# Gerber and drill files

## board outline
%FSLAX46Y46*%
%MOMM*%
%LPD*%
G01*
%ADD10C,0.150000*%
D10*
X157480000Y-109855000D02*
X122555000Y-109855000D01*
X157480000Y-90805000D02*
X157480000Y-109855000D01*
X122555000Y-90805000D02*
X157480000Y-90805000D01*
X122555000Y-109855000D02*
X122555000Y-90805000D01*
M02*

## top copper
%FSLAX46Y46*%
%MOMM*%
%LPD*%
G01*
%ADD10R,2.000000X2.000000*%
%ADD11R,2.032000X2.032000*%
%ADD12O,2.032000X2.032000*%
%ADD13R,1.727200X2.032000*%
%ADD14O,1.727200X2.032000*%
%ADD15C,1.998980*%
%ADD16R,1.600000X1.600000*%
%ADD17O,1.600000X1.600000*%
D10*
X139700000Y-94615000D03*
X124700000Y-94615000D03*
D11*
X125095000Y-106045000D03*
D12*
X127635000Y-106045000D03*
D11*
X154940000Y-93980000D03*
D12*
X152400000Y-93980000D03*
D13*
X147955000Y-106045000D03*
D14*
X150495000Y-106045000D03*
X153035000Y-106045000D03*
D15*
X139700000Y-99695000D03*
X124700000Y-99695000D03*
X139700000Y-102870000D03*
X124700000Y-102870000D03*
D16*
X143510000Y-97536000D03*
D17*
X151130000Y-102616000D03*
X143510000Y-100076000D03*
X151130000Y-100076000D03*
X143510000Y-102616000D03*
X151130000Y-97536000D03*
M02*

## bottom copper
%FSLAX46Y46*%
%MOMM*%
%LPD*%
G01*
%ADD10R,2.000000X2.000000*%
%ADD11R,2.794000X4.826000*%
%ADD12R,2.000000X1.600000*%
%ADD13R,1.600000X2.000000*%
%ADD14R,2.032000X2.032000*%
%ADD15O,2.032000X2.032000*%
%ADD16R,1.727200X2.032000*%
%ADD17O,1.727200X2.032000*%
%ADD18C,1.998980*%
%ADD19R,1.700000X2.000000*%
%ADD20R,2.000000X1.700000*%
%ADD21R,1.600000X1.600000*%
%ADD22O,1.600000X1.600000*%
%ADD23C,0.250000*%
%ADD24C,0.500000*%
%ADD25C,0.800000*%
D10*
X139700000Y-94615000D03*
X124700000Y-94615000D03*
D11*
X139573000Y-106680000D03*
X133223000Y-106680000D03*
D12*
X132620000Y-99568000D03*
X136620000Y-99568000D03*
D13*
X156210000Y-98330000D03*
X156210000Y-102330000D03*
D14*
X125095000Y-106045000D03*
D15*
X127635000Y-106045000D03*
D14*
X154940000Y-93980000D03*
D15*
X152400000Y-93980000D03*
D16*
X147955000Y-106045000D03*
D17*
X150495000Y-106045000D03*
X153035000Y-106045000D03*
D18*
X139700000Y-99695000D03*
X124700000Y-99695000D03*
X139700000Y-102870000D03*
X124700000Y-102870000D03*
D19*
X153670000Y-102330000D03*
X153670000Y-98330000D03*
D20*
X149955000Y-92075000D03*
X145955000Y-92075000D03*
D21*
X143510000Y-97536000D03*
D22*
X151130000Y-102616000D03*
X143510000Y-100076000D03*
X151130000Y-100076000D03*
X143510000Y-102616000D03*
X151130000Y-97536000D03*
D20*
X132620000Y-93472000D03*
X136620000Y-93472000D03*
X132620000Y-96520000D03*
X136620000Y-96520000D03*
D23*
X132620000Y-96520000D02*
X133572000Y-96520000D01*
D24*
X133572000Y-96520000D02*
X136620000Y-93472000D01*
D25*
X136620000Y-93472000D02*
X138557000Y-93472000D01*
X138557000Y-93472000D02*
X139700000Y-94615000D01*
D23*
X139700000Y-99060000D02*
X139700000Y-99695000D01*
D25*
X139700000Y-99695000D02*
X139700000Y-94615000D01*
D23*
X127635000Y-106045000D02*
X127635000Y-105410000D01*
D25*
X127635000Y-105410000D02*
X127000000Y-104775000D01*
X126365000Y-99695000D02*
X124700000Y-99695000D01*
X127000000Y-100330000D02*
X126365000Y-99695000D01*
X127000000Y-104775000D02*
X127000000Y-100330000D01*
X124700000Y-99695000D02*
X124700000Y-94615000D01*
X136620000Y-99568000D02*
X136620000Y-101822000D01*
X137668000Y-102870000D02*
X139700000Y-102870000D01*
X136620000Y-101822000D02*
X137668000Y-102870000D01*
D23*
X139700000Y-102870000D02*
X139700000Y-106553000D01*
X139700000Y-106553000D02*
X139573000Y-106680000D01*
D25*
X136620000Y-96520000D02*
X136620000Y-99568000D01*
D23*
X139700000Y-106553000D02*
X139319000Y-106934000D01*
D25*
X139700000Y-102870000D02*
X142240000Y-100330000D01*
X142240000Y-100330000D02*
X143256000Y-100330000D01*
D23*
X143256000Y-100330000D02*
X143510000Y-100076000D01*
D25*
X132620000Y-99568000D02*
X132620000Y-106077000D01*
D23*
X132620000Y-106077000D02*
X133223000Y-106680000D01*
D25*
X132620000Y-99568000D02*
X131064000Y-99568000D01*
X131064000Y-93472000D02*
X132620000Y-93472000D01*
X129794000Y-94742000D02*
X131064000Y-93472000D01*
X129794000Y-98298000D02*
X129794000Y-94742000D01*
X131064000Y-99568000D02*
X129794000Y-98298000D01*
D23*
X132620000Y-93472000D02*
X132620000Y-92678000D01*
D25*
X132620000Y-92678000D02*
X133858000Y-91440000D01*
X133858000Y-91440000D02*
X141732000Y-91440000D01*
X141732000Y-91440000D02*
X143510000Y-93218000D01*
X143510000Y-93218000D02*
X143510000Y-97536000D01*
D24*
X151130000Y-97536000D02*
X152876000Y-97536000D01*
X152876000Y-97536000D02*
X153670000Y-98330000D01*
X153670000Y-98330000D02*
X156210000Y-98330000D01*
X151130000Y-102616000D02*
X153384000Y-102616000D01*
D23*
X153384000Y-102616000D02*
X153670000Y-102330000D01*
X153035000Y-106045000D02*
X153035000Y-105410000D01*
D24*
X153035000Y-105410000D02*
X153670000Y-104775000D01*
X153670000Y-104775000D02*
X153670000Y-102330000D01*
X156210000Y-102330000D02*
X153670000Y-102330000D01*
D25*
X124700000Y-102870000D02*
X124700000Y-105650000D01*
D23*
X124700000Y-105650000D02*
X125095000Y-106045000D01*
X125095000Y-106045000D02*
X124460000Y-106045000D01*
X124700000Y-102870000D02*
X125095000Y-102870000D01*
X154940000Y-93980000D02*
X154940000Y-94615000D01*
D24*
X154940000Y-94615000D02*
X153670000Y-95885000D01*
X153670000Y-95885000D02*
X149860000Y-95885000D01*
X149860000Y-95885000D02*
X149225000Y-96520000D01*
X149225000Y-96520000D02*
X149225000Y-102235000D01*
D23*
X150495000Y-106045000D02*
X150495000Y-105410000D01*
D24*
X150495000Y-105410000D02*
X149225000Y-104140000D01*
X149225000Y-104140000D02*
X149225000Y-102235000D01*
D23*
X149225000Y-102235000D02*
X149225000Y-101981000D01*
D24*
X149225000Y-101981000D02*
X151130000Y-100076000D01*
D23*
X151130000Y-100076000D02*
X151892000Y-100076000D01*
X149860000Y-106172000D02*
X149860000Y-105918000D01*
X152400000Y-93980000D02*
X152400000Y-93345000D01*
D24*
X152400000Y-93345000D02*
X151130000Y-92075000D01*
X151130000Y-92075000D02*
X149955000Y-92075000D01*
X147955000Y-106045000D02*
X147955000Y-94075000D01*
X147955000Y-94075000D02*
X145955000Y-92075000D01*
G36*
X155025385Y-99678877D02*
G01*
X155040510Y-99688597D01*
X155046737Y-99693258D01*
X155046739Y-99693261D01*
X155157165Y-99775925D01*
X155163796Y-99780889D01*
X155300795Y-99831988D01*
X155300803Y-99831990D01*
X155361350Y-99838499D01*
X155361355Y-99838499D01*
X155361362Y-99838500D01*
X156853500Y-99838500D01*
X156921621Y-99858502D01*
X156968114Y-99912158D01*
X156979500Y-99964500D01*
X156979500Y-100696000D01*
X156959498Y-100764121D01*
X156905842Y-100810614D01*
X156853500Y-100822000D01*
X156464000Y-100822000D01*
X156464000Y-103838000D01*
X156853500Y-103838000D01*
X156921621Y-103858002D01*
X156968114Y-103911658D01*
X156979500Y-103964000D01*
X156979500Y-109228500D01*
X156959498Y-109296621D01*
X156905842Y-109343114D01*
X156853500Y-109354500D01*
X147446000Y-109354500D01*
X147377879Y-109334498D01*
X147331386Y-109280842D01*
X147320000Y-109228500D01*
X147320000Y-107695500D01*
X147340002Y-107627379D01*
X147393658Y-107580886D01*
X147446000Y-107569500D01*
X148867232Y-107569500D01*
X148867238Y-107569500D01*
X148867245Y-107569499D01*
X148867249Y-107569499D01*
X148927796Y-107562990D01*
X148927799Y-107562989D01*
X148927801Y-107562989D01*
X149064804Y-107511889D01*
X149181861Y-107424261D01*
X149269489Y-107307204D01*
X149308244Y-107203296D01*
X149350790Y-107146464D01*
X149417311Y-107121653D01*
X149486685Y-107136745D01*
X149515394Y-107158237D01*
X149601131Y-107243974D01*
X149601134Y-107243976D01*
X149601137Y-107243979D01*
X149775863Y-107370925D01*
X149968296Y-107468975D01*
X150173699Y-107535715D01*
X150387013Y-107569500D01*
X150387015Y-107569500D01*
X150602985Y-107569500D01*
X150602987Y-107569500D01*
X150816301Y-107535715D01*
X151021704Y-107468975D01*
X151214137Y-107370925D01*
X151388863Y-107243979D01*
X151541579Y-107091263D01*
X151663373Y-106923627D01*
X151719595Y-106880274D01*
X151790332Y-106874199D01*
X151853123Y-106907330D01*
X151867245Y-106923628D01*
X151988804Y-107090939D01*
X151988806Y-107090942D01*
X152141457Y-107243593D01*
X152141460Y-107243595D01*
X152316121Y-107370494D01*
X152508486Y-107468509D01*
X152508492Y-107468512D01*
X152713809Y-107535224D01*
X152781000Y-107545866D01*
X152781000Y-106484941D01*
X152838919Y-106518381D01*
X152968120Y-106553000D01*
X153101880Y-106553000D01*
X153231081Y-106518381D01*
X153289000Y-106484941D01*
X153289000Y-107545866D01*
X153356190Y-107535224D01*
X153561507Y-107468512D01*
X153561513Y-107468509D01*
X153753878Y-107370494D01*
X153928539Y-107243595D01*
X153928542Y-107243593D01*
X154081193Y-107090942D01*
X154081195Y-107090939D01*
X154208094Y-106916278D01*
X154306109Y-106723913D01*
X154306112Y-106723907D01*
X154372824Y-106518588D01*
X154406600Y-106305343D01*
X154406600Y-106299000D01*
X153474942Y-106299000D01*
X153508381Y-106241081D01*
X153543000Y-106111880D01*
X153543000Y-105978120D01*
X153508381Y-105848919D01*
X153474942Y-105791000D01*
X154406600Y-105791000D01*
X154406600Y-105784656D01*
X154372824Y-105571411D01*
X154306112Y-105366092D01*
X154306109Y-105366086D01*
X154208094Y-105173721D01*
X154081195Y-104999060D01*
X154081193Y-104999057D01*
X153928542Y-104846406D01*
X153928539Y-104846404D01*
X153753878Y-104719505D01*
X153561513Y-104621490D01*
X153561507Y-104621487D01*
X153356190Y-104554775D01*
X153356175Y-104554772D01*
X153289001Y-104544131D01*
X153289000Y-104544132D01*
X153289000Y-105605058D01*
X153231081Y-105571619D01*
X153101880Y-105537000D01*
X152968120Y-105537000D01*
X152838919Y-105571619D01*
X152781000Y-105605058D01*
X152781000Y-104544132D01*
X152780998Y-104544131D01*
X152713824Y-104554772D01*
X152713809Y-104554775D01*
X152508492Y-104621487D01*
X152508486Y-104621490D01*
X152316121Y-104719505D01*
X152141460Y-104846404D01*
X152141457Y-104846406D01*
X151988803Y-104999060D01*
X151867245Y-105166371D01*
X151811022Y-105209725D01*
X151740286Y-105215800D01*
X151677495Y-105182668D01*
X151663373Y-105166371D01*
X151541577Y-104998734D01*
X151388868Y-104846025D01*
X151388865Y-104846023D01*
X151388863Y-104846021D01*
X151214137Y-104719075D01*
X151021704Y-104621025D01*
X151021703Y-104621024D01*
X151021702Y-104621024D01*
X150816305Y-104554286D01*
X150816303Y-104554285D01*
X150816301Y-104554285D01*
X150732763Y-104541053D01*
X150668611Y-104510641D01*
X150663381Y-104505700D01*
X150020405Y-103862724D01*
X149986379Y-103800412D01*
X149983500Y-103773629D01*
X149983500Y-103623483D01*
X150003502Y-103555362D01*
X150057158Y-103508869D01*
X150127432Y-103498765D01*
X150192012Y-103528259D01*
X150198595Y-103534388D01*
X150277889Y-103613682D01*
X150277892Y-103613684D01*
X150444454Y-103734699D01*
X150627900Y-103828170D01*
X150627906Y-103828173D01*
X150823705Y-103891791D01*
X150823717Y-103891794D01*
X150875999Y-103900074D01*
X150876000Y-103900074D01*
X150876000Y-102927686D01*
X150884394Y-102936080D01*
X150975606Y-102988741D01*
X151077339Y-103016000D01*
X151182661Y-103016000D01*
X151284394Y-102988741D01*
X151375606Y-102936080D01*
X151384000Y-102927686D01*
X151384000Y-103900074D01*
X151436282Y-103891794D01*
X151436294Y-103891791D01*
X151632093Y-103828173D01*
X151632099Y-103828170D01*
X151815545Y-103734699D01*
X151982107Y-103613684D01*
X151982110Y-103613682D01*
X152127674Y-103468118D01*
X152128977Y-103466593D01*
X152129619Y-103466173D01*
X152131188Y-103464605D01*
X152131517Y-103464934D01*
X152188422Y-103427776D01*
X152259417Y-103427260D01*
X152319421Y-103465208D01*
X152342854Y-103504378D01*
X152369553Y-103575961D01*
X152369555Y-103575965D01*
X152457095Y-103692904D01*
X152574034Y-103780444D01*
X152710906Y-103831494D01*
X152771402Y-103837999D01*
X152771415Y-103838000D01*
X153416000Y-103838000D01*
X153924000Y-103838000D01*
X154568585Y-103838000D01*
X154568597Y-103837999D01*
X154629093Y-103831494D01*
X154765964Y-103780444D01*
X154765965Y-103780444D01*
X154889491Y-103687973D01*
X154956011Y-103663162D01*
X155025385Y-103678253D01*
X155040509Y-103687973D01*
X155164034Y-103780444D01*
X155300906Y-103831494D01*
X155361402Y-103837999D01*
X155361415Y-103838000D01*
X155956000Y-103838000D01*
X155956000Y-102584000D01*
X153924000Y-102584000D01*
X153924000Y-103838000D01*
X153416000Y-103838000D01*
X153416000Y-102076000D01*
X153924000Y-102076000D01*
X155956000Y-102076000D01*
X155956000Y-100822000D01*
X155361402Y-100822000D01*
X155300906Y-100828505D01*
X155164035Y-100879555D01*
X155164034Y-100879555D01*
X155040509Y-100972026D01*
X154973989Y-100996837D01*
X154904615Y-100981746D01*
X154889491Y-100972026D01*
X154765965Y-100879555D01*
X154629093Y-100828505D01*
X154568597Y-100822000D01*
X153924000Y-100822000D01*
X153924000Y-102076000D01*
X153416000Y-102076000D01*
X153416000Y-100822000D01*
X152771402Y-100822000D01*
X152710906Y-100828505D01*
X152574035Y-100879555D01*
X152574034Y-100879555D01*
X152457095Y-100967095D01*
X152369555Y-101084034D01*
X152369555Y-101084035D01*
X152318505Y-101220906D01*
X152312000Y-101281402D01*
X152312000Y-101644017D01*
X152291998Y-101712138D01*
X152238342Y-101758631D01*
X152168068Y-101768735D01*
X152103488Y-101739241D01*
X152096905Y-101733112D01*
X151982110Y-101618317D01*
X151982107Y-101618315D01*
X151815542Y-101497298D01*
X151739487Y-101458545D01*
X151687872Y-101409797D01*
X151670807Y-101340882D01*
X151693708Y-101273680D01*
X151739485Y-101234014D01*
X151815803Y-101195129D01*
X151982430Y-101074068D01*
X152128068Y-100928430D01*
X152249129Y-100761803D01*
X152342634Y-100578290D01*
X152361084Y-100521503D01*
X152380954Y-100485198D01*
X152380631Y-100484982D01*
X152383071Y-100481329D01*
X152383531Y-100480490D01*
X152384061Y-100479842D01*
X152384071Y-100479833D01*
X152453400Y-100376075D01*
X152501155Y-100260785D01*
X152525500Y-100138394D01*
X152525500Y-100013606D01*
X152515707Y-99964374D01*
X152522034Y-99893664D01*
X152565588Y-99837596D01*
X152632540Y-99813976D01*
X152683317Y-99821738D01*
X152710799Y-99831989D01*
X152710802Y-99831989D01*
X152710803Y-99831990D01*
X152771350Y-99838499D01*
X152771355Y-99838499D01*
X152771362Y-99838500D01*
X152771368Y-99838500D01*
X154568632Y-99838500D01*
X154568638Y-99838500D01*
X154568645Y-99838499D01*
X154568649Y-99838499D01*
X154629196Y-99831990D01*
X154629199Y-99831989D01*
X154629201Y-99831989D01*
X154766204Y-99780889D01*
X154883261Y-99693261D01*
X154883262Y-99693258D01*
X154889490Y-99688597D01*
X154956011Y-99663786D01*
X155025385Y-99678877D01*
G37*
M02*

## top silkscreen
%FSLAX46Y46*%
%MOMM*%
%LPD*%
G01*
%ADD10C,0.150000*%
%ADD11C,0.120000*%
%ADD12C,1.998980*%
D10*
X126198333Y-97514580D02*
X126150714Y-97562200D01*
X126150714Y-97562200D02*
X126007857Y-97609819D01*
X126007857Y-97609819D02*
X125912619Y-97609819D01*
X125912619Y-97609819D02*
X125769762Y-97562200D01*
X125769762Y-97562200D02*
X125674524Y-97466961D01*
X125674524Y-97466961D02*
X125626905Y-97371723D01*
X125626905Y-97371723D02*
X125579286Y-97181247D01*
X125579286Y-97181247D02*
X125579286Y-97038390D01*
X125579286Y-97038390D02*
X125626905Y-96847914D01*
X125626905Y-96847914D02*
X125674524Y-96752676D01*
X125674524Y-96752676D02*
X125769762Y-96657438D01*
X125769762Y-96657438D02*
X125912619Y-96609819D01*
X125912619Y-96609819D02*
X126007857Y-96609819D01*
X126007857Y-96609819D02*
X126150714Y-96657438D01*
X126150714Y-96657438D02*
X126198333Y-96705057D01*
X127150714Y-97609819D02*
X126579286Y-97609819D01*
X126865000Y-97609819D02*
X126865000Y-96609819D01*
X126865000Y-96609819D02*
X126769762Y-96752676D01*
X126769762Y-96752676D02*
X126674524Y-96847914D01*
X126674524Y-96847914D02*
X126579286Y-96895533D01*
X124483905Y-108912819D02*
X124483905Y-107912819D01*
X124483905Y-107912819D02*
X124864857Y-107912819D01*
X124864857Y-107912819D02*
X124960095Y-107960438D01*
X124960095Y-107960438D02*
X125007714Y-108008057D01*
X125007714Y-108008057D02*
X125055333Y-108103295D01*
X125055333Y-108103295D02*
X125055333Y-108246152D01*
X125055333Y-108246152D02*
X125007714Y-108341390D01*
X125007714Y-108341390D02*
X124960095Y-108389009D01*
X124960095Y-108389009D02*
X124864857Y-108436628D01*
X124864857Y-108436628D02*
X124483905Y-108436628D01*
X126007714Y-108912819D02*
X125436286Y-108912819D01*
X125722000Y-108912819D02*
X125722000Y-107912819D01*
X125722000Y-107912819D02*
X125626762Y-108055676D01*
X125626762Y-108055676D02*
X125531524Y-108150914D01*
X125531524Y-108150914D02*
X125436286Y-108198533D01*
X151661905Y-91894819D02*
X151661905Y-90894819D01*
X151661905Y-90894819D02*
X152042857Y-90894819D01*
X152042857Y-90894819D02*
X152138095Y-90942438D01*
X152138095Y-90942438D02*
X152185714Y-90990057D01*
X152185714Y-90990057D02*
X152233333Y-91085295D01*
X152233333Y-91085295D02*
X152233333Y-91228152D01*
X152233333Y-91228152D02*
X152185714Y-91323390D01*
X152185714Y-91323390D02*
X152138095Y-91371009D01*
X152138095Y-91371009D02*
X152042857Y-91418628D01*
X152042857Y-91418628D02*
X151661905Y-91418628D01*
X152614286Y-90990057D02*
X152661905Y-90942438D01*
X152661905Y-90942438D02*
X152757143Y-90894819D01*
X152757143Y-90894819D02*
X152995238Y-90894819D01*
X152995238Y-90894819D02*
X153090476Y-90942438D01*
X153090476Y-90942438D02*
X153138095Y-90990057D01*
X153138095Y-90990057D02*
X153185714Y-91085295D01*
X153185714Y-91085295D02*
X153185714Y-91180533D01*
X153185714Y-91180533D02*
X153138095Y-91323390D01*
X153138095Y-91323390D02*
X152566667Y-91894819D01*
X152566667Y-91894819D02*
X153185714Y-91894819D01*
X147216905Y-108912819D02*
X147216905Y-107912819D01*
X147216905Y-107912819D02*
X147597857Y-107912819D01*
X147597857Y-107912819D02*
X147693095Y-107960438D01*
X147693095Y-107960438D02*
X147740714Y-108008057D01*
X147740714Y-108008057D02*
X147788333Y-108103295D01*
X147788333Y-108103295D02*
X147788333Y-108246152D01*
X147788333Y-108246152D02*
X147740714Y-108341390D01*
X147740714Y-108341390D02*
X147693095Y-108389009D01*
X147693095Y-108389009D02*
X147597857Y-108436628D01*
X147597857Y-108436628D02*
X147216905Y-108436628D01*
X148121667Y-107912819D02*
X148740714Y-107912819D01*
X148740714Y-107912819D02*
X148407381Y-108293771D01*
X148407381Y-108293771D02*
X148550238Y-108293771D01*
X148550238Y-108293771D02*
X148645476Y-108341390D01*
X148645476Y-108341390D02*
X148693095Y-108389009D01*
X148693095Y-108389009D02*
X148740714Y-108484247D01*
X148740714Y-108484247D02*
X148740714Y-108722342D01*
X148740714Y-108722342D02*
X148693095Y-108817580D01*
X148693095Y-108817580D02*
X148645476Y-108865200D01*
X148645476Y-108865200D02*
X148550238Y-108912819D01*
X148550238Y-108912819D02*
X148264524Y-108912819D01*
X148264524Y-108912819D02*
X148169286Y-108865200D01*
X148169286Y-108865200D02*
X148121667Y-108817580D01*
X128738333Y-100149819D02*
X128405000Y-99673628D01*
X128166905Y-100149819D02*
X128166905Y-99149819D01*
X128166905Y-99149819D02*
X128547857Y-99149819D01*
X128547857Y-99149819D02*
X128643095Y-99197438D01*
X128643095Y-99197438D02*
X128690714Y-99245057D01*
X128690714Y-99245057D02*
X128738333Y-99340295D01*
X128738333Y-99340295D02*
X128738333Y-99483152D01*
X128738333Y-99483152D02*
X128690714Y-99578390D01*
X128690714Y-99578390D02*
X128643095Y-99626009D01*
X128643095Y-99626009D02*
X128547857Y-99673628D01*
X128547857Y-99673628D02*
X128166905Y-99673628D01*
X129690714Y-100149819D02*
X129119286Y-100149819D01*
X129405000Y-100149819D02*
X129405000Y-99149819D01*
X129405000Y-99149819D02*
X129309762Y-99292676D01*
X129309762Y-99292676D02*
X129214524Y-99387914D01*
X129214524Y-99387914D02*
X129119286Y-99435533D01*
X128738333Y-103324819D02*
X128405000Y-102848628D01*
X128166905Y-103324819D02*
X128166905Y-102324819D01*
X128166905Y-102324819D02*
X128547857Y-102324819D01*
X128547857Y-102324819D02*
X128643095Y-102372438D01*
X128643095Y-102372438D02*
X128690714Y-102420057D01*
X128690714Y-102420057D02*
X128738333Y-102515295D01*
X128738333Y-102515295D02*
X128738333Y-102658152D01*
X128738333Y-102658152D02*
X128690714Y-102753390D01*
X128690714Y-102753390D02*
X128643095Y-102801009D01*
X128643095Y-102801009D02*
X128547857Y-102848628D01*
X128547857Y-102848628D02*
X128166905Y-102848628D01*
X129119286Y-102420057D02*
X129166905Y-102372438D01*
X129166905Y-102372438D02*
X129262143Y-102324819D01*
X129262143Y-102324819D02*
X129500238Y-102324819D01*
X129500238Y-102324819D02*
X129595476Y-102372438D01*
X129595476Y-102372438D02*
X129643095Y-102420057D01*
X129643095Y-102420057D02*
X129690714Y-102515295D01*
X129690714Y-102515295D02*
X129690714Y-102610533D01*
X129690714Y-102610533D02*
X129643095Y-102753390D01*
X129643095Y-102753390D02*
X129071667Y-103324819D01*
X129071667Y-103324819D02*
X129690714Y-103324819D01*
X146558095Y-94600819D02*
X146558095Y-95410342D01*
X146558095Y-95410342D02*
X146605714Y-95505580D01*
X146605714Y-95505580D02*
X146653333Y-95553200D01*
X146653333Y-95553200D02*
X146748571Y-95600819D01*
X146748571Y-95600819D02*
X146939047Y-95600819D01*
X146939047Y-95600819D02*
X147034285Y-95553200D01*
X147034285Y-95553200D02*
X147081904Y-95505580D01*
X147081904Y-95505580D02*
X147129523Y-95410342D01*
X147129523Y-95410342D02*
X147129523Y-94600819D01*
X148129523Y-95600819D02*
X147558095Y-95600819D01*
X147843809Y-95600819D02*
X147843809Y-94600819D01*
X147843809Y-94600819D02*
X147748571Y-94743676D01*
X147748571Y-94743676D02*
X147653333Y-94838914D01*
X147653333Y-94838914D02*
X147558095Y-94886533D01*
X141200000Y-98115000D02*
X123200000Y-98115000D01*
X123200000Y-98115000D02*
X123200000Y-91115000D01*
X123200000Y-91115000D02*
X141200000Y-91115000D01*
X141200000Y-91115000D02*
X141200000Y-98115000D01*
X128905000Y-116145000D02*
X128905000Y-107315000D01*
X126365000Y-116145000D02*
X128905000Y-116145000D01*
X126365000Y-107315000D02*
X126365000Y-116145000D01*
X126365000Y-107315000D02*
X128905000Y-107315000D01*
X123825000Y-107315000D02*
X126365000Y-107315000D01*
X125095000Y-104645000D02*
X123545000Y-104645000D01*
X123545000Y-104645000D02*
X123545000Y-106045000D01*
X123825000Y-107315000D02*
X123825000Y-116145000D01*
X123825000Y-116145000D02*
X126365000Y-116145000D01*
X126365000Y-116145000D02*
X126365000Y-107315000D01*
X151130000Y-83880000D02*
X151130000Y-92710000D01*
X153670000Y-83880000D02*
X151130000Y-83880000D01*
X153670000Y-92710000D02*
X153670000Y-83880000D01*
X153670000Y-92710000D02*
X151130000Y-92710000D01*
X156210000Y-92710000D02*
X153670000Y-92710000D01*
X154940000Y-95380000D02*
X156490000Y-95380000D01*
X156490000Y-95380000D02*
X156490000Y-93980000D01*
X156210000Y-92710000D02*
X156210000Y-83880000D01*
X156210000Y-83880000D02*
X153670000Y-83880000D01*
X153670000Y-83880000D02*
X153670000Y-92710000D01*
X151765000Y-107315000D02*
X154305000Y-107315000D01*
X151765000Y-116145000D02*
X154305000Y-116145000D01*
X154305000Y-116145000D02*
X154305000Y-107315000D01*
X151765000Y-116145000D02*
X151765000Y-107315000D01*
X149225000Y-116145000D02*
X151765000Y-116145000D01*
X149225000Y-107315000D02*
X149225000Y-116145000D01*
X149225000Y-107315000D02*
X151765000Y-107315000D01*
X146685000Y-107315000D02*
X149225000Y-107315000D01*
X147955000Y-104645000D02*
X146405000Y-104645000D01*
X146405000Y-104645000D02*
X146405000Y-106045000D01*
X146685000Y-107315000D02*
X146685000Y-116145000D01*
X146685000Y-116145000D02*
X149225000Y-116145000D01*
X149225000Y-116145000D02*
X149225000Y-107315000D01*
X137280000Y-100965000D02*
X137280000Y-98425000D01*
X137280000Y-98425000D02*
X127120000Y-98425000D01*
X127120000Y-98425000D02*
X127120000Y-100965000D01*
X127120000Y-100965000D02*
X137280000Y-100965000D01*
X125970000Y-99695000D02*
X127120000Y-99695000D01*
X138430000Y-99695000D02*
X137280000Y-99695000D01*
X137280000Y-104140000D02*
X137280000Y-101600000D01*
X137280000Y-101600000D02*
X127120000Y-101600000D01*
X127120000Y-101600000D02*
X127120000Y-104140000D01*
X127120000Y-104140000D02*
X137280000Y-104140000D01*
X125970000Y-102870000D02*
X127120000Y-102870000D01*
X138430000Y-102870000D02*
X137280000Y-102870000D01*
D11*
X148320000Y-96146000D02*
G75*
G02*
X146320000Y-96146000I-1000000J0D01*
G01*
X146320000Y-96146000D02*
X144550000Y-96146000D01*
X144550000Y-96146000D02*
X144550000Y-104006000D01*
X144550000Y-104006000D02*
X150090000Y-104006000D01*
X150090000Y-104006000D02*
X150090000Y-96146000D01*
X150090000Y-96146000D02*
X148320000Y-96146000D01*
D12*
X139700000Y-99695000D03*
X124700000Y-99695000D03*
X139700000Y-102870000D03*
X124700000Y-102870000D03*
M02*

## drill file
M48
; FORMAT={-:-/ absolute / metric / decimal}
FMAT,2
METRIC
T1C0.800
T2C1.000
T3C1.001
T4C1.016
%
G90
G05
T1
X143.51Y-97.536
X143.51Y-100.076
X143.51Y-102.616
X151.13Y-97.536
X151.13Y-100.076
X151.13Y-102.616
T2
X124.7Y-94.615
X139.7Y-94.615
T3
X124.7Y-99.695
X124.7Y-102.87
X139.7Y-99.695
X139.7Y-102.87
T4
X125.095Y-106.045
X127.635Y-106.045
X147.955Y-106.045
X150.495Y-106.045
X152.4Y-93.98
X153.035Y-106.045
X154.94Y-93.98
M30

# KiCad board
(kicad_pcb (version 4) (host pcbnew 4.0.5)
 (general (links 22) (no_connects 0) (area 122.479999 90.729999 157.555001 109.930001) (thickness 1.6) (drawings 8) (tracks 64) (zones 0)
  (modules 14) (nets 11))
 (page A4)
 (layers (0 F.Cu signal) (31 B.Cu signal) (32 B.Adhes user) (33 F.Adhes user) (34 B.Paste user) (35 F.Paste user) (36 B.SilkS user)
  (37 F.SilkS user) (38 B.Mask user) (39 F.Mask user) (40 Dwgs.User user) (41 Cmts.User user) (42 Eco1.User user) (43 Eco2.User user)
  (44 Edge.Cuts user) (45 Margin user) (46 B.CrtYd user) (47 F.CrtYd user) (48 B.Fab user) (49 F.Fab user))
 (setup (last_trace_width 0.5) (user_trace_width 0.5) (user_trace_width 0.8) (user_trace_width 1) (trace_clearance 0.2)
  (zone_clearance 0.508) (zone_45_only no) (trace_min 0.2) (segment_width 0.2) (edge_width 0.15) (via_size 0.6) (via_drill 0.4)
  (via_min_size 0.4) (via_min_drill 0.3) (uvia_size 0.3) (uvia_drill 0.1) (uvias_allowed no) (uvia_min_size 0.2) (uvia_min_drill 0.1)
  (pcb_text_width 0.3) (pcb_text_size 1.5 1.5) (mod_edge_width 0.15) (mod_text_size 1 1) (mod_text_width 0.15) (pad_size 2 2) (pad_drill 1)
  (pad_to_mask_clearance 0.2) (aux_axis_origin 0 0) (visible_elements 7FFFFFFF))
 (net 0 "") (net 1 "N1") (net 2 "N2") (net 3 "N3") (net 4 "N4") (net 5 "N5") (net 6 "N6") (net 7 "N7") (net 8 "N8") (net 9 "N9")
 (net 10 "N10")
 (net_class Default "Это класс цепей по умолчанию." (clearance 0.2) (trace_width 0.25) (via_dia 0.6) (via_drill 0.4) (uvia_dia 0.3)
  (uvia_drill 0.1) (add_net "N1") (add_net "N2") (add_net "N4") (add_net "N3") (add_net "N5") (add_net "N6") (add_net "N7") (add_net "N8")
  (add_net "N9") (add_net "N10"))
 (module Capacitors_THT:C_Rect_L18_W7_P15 (layer F.Cu) (at 139.7 94.615 180)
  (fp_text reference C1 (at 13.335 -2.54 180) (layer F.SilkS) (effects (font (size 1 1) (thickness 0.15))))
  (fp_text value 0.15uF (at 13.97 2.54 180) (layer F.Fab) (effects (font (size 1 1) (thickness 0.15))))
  (fp_line (start -1.5 -3.5) (end 16.5 -3.5) (layer F.SilkS) (width 0.15))
  (fp_line (start 16.5 -3.5) (end 16.5 3.5) (layer F.SilkS) (width 0.15))
  (fp_line (start 16.5 3.5) (end -1.5 3.5) (layer F.SilkS) (width 0.15))
  (fp_line (start -1.5 3.5) (end -1.5 -3.5) (layer F.SilkS) (width 0.15))
  (pad 1 thru_hole rect (at 0 0 180) (size 2 2) (drill 1) (layers *.Cu *.Mask) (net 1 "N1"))
  (pad 2 thru_hole rect (at 15 0 180) (size 2 2) (drill 1) (layers *.Cu *.Mask) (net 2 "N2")))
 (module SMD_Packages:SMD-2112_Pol (layer B.Cu) (at 136.398 106.68)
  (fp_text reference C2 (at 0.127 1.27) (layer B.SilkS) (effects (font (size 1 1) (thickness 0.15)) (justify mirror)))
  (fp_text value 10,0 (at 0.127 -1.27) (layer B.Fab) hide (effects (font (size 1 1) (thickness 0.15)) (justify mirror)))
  (pad 2 smd rect (at 3.175 0) (size 2.794 4.826) (layers B.Cu B.Paste B.Mask) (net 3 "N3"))
  (pad 1 smd rect (at -3.175 0) (size 2.794 4.826) (layers B.Cu B.Paste B.Mask) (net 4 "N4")))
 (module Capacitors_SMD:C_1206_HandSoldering (layer B.Cu) (at 134.62 99.568)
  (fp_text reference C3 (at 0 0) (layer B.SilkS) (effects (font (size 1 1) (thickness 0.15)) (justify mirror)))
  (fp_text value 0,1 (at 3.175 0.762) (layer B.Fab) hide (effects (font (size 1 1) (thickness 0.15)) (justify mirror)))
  (pad 1 smd rect (at -2 0) (size 2 1.6) (layers B.Cu B.Paste B.Mask) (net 4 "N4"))
  (pad 2 smd rect (at 2 0) (size 2 1.6) (layers B.Cu B.Paste B.Mask) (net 3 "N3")))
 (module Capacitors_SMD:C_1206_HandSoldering (layer B.Cu) (at 156.21 100.33 270)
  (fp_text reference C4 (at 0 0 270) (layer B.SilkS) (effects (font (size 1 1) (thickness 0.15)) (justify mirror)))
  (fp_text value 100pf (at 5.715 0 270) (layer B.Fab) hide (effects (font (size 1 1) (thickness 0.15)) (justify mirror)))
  (pad 1 smd rect (at -2 0 270) (size 2 1.6) (layers B.Cu B.Paste B.Mask) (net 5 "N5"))
  (pad 2 smd rect (at 2 0 270) (size 2 1.6) (layers B.Cu B.Paste B.Mask) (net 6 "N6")))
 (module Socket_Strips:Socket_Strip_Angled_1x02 (layer F.Cu) (at 125.095 106.045)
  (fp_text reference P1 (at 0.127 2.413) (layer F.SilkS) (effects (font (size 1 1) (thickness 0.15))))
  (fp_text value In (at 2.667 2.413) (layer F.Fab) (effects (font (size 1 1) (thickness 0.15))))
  (fp_line (start 3.81 10.1) (end 3.81 1.27) (layer F.SilkS) (width 0.15))
  (fp_line (start 1.27 10.1) (end 3.81 10.1) (layer F.SilkS) (width 0.15))
  (fp_line (start 1.27 1.27) (end 1.27 10.1) (layer F.SilkS) (width 0.15))
  (fp_line (start 1.27 1.27) (end 3.81 1.27) (layer F.SilkS) (width 0.15))
  (fp_line (start -1.27 1.27) (end 1.27 1.27) (layer F.SilkS) (width 0.15))
  (fp_line (start 0 -1.4) (end -1.55 -1.4) (layer F.SilkS) (width 0.15))
  (fp_line (start -1.55 -1.4) (end -1.55 0) (layer F.SilkS) (width 0.15))
  (fp_line (start -1.27 1.27) (end -1.27 10.1) (layer F.SilkS) (width 0.15))
  (fp_line (start -1.27 10.1) (end 1.27 10.1) (layer F.SilkS) (width 0.15))
  (fp_line (start 1.27 10.1) (end 1.27 1.27) (layer F.SilkS) (width 0.15))
  (pad 1 thru_hole rect (at 0 0) (size 2.032 2.032) (drill 1.016) (layers *.Cu *.Mask) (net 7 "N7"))
  (pad 2 thru_hole oval (at 2.54 0) (size 2.032 2.032) (drill 1.016) (layers *.Cu *.Mask) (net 2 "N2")))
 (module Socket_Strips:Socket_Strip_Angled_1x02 (layer F.Cu) (at 154.94 93.98 180)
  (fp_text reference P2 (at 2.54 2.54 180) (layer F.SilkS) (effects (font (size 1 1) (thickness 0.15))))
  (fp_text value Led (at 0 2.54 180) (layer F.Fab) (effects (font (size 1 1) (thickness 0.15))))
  (fp_line (start 3.81 10.1) (end 3.81 1.27) (layer F.SilkS) (width 0.15))
  (fp_line (start 1.27 10.1) (end 3.81 10.1) (layer F.SilkS) (width 0.15))
  (fp_line (start 1.27 1.27) (end 1.27 10.1) (layer F.SilkS) (width 0.15))
  (fp_line (start 1.27 1.27) (end 3.81 1.27) (layer F.SilkS) (width 0.15))
  (fp_line (start -1.27 1.27) (end 1.27 1.27) (layer F.SilkS) (width 0.15))
  (fp_line (start 0 -1.4) (end -1.55 -1.4) (layer F.SilkS) (width 0.15))
  (fp_line (start -1.55 -1.4) (end -1.55 0) (layer F.SilkS) (width 0.15))
  (fp_line (start -1.27 1.27) (end -1.27 10.1) (layer F.SilkS) (width 0.15))
  (fp_line (start -1.27 10.1) (end 1.27 10.1) (layer F.SilkS) (width 0.15))
  (fp_line (start 1.27 10.1) (end 1.27 1.27) (layer F.SilkS) (width 0.15))
  (pad 1 thru_hole rect (at 0 0 180) (size 2.032 2.032) (drill 1.016) (layers *.Cu *.Mask) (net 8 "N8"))
  (pad 2 thru_hole oval (at 2.54 0 180) (size 2.032 2.032) (drill 1.016) (layers *.Cu *.Mask) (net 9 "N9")))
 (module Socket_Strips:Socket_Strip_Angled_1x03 (layer F.Cu) (at 147.955 106.045)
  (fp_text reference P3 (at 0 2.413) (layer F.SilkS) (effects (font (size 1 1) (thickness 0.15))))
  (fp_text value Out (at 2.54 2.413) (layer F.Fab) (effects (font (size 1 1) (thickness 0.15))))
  (fp_line (start 3.81 1.27) (end 6.35 1.27) (layer F.SilkS) (width 0.15))
  (fp_line (start 3.81 10.1) (end 6.35 10.1) (layer F.SilkS) (width 0.15))
  (fp_line (start 6.35 10.1) (end 6.35 1.27) (layer F.SilkS) (width 0.15))
  (fp_line (start 3.81 10.1) (end 3.81 1.27) (layer F.SilkS) (width 0.15))
  (fp_line (start 1.27 10.1) (end 3.81 10.1) (layer F.SilkS) (width 0.15))
  (fp_line (start 1.27 1.27) (end 1.27 10.1) (layer F.SilkS) (width 0.15))
  (fp_line (start 1.27 1.27) (end 3.81 1.27) (layer F.SilkS) (width 0.15))
  (fp_line (start -1.27 1.27) (end 1.27 1.27) (layer F.SilkS) (width 0.15))
  (fp_line (start 0 -1.4) (end -1.55 -1.4) (layer F.SilkS) (width 0.15))
  (fp_line (start -1.55 -1.4) (end -1.55 0) (layer F.SilkS) (width 0.15))
  (fp_line (start -1.27 1.27) (end -1.27 10.1) (layer F.SilkS) (width 0.15))
  (fp_line (start -1.27 10.1) (end 1.27 10.1) (layer F.SilkS) (width 0.15))
  (fp_line (start 1.27 10.1) (end 1.27 1.27) (layer F.SilkS) (width 0.15))
  (pad 1 thru_hole rect (at 0 0) (size 1.7272 2.032) (drill 1.016) (layers *.Cu *.Mask) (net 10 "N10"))
  (pad 2 thru_hole oval (at 2.54 0) (size 1.7272 2.032) (drill 1.016) (layers *.Cu *.Mask) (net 8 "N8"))
  (pad 3 thru_hole oval (at 5.08 0) (size 1.7272 2.032) (drill 1.016) (layers *.Cu *.Mask) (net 6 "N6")))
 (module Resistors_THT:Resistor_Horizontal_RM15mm (layer F.Cu) (at 139.7 99.695 180)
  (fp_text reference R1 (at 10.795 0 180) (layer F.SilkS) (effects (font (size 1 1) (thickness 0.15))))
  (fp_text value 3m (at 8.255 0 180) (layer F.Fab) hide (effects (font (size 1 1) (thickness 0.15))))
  (fp_line (start 2.42 -1.27) (end 2.42 1.27) (layer F.SilkS) (width 0.15))
  (fp_line (start 2.42 1.27) (end 12.58 1.27) (layer F.SilkS) (width 0.15))
  (fp_line (start 12.58 1.27) (end 12.58 -1.27) (layer F.SilkS) (width 0.15))
  (fp_line (start 12.58 -1.27) (end 2.42 -1.27) (layer F.SilkS) (width 0.15))
  (fp_line (start 13.73 0) (end 12.58 0) (layer F.SilkS) (width 0.15))
  (fp_line (start 1.27 0) (end 2.42 0) (layer F.SilkS) (width 0.15))
  (pad 1 thru_hole circle (at 0 0 180) (size 1.99898 1.99898) (drill 1.00076) (layers *.Cu *.SilkS *.Mask) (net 1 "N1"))
  (pad 2 thru_hole circle (at 15 0 180) (size 1.99898 1.99898) (drill 1.00076) (layers *.Cu *.SilkS *.Mask) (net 2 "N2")))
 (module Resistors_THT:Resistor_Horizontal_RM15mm (layer F.Cu) (at 139.7 102.87 180)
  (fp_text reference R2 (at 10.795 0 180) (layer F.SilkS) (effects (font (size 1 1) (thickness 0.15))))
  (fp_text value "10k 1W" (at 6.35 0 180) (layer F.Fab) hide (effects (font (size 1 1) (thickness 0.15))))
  (fp_line (start 2.42 -1.27) (end 2.42 1.27) (layer F.SilkS) (width 0.15))
  (fp_line (start 2.42 1.27) (end 12.58 1.27) (layer F.SilkS) (width 0.15))
  (fp_line (start 12.58 1.27) (end 12.58 -1.27) (layer F.SilkS) (width 0.15))
  (fp_line (start 12.58 -1.27) (end 2.42 -1.27) (layer F.SilkS) (width 0.15))
  (fp_line (start 13.73 0) (end 12.58 0) (layer F.SilkS) (width 0.15))
  (fp_line (start 1.27 0) (end 2.42 0) (layer F.SilkS) (width 0.15))
  (pad 1 thru_hole circle (at 0 0 180) (size 1.99898 1.99898) (drill 1.00076) (layers *.Cu *.SilkS *.Mask) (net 3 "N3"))
  (pad 2 thru_hole circle (at 15 0 180) (size 1.99898 1.99898) (drill 1.00076) (layers *.Cu *.SilkS *.Mask) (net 7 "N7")))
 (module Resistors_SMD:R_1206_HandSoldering (layer B.Cu) (at 153.67 100.33 90)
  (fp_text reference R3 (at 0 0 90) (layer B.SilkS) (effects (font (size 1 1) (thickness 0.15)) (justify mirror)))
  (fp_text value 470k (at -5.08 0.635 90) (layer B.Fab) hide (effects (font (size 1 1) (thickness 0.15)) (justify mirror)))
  (pad 1 smd rect (at -2 0 90) (size 2 1.7) (layers B.Cu B.Paste B.Mask) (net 6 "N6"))
  (pad 2 smd rect (at 2 0 90) (size 2 1.7) (layers B.Cu B.Paste B.Mask) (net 5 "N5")))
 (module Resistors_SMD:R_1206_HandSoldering (layer B.Cu) (at 147.955 92.075 180)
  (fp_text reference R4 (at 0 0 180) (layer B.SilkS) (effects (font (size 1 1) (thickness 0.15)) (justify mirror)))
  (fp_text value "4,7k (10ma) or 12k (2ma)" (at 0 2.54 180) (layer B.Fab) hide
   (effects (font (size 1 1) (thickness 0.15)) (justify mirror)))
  (pad 1 smd rect (at -2 0 180) (size 2 1.7) (layers B.Cu B.Paste B.Mask) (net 9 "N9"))
  (pad 2 smd rect (at 2 0 180) (size 2 1.7) (layers B.Cu B.Paste B.Mask) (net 10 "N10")))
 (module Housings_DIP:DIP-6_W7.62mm (layer F.Cu) (at 143.51 97.536)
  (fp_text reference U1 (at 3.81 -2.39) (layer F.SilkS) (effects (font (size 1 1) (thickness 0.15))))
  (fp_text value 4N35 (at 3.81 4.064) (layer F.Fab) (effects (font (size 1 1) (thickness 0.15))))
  (fp_arc (start 3.81 -1.39) (end 2.81 -1.39) (angle -180) (layer F.SilkS) (width 0.12))
  (fp_line (start 2.81 -1.39) (end 1.04 -1.39) (layer F.SilkS) (width 0.12))
  (fp_line (start 1.04 -1.39) (end 1.04 6.47) (layer F.SilkS) (width 0.12))
  (fp_line (start 1.04 6.47) (end 6.58 6.47) (layer F.SilkS) (width 0.12))
  (fp_line (start 6.58 6.47) (end 6.58 -1.39) (layer F.SilkS) (width 0.12))
  (fp_line (start 6.58 -1.39) (end 4.81 -1.39) (layer F.SilkS) (width 0.12))
  (pad 1 thru_hole rect (at 0 0) (size 1.6 1.6) (drill 0.8) (layers *.Cu *.Mask) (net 4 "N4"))
  (pad 4 thru_hole oval (at 7.62 5.08) (size 1.6 1.6) (drill 0.8) (layers *.Cu *.Mask) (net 6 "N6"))
  (pad 2 thru_hole oval (at 0 2.54) (size 1.6 1.6) (drill 0.8) (layers *.Cu *.Mask) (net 3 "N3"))
  (pad 5 thru_hole oval (at 7.62 2.54) (size 1.6 1.6) (drill 0.8) (layers *.Cu *.Mask) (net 8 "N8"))
  (pad 3 thru_hole oval (at 0 5.08) (size 1.6 1.6) (drill 0.8) (layers *.Cu *.Mask))
  (pad 6 thru_hole oval (at 7.62 0) (size 1.6 1.6) (drill 0.8) (layers *.Cu *.Mask) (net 5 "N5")))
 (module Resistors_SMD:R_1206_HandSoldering (layer B.Cu) (at 134.62 93.472)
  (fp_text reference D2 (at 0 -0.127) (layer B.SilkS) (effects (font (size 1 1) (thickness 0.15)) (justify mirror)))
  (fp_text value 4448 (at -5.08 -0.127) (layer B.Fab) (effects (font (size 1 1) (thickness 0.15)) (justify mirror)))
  (pad 1 smd rect (at -2 0) (size 2 1.7) (layers B.Cu B.Paste B.Mask) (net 4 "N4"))
  (pad 2 smd rect (at 2 0) (size 2 1.7) (layers B.Cu B.Paste B.Mask) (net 1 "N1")))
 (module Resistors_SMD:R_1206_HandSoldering (layer B.Cu) (at 134.62 96.52)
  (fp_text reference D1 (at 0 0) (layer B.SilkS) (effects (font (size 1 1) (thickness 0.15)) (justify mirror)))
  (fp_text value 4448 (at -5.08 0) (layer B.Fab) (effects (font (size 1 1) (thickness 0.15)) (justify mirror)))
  (pad 1 smd rect (at -2 0) (size 2 1.7) (layers B.Cu B.Paste B.Mask) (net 1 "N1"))
  (pad 2 smd rect (at 2 0) (size 2 1.7) (layers B.Cu B.Paste B.Mask) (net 3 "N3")))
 (gr_line (start 157.48 109.855) (end 122.555 109.855) (angle 90) (layer Edge.Cuts) (width 0.15))
 (gr_line (start 157.48 90.805) (end 157.48 109.855) (angle 90) (layer Edge.Cuts) (width 0.15))
 (gr_line (start 122.555 90.805) (end 157.48 90.805) (angle 90) (layer Edge.Cuts) (width 0.15))
 (gr_line (start 122.555 109.855) (end 122.555 90.805) (angle 90) (layer Edge.Cuts) (width 0.15))
 (segment (start 132.62 96.52) (end 133.572 96.52) (width 0.25) (layer B.Cu) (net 1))
 (segment (start 133.572 96.52) (end 136.62 93.472) (width 0.5) (layer B.Cu) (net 1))
 (segment (start 136.62 93.472) (end 138.557 93.472) (width 0.8) (layer B.Cu) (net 1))
 (segment (start 138.557 93.472) (end 139.7 94.615) (width 0.8) (layer B.Cu) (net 1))
 (segment (start 139.7 99.06) (end 139.7 99.695) (width 0.25) (layer B.Cu) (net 1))
 (segment (start 139.7 99.695) (end 139.7 94.615) (width 0.8) (layer B.Cu) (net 1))
 (segment (start 127.635 106.045) (end 127.635 105.41) (width 0.25) (layer B.Cu) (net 2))
 (segment (start 127.635 105.41) (end 127 104.775) (width 0.8) (layer B.Cu) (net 2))
 (segment (start 126.365 99.695) (end 124.7 99.695) (width 0.8) (layer B.Cu) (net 2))
 (segment (start 127 100.33) (end 126.365 99.695) (width 0.8) (layer B.Cu) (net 2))
 (segment (start 127 104.775) (end 127 100.33) (width 0.8) (layer B.Cu) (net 2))
 (segment (start 124.7 99.695) (end 124.7 94.615) (width 0.8) (layer B.Cu) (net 2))
 (segment (start 136.62 99.568) (end 136.62 101.822) (width 0.8) (layer B.Cu) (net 3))
 (segment (start 137.668 102.87) (end 139.7 102.87) (width 0.8) (layer B.Cu) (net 3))
 (segment (start 136.62 101.822) (end 137.668 102.87) (width 0.8) (layer B.Cu) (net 3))
 (segment (start 139.7 102.87) (end 139.7 106.553) (width 0.25) (layer B.Cu) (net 3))
 (segment (start 139.7 106.553) (end 139.573 106.68) (width 0.25) (layer B.Cu) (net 3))
 (segment (start 136.62 96.52) (end 136.62 99.568) (width 0.8) (layer B.Cu) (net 3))
 (segment (start 139.7 106.553) (end 139.319 106.934) (width 0.25) (layer B.Cu) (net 3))
 (segment (start 139.7 102.87) (end 142.24 100.33) (width 0.8) (layer B.Cu) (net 3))
 (segment (start 142.24 100.33) (end 143.256 100.33) (width 0.8) (layer B.Cu) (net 3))
 (segment (start 143.256 100.33) (end 143.51 100.076) (width 0.25) (layer B.Cu) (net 3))
 (segment (start 132.62 99.568) (end 132.62 106.077) (width 0.8) (layer B.Cu) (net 4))
 (segment (start 132.62 106.077) (end 133.223 106.68) (width 0.25) (layer B.Cu) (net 4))
 (segment (start 132.62 99.568) (end 131.064 99.568) (width 0.8) (layer B.Cu) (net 4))
 (segment (start 131.064 93.472) (end 132.62 93.472) (width 0.8) (layer B.Cu) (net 4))
 (segment (start 129.794 94.742) (end 131.064 93.472) (width 0.8) (layer B.Cu) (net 4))
 (segment (start 129.794 98.298) (end 129.794 94.742) (width 0.8) (layer B.Cu) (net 4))
 (segment (start 131.064 99.568) (end 129.794 98.298) (width 0.8) (layer B.Cu) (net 4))
 (segment (start 132.62 93.472) (end 132.62 92.678) (width 0.25) (layer B.Cu) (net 4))
 (segment (start 132.62 92.678) (end 133.858 91.44) (width 0.8) (layer B.Cu) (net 4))
 (segment (start 133.858 91.44) (end 141.732 91.44) (width 0.8) (layer B.Cu) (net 4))
 (segment (start 141.732 91.44) (end 143.51 93.218) (width 0.8) (layer B.Cu) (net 4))
 (segment (start 143.51 93.218) (end 143.51 97.536) (width 0.8) (layer B.Cu) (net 4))
 (segment (start 151.13 97.536) (end 152.876 97.536) (width 0.5) (layer B.Cu) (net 5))
 (segment (start 152.876 97.536) (end 153.67 98.33) (width 0.5) (layer B.Cu) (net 5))
 (segment (start 153.67 98.33) (end 156.21 98.33) (width 0.5) (layer B.Cu) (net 5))
 (segment (start 151.13 102.616) (end 153.384 102.616) (width 0.5) (layer B.Cu) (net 6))
 (segment (start 153.384 102.616) (end 153.67 102.33) (width 0.25) (layer B.Cu) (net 6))
 (segment (start 153.035 106.045) (end 153.035 105.41) (width 0.25) (layer B.Cu) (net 6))
 (segment (start 153.035 105.41) (end 153.67 104.775) (width 0.5) (layer B.Cu) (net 6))
 (segment (start 153.67 104.775) (end 153.67 102.33) (width 0.5) (layer B.Cu) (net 6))
 (segment (start 156.21 102.33) (end 153.67 102.33) (width 0.5) (layer B.Cu) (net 6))
 (segment (start 124.7 102.87) (end 124.7 105.65) (width 0.8) (layer B.Cu) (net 7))
 (segment (start 124.7 105.65) (end 125.095 106.045) (width 0.25) (layer B.Cu) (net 7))
 (segment (start 125.095 106.045) (end 124.46 106.045) (width 0.25) (layer B.Cu) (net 7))
 (segment (start 124.7 102.87) (end 125.095 102.87) (width 0.25) (layer B.Cu) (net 7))
 (segment (start 154.94 93.98) (end 154.94 94.615) (width 0.25) (layer B.Cu) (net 8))
 (segment (start 154.94 94.615) (end 153.67 95.885) (width 0.5) (layer B.Cu) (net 8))
 (segment (start 153.67 95.885) (end 149.86 95.885) (width 0.5) (layer B.Cu) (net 8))
 (segment (start 149.86 95.885) (end 149.225 96.52) (width 0.5) (layer B.Cu) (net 8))
 (segment (start 149.225 96.52) (end 149.225 102.235) (width 0.5) (layer B.Cu) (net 8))
 (segment (start 150.495 106.045) (end 150.495 105.41) (width 0.25) (layer B.Cu) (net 8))
 (segment (start 150.495 105.41) (end 149.225 104.14) (width 0.5) (layer B.Cu) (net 8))
 (segment (start 149.225 104.14) (end 149.225 102.235) (width 0.5) (layer B.Cu) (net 8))
 (segment (start 149.225 102.235) (end 149.225 101.981) (width 0.25) (layer B.Cu) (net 8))
 (segment (start 149.225 101.981) (end 151.13 100.076) (width 0.5) (layer B.Cu) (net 8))
 (segment (start 151.13 100.076) (end 151.892 100.076) (width 0.25) (layer B.Cu) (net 8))
 (segment (start 149.86 106.172) (end 149.86 105.918) (width 0.25) (layer B.Cu) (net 8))
 (segment (start 152.4 93.98) (end 152.4 93.345) (width 0.25) (layer B.Cu) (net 9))
 (segment (start 152.4 93.345) (end 151.13 92.075) (width 0.5) (layer B.Cu) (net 9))
 (segment (start 151.13 92.075) (end 149.955 92.075) (width 0.5) (layer B.Cu) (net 9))
 (segment (start 147.955 106.045) (end 147.955 94.075) (width 0.5) (layer B.Cu) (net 10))
 (segment (start 147.955 94.075) (end 145.955 92.075) (width 0.5) (layer B.Cu) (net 10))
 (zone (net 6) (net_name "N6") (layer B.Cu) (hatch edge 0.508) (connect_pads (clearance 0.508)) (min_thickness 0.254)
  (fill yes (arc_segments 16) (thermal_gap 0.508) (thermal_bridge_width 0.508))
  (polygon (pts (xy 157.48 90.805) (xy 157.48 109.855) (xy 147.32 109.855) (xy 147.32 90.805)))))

